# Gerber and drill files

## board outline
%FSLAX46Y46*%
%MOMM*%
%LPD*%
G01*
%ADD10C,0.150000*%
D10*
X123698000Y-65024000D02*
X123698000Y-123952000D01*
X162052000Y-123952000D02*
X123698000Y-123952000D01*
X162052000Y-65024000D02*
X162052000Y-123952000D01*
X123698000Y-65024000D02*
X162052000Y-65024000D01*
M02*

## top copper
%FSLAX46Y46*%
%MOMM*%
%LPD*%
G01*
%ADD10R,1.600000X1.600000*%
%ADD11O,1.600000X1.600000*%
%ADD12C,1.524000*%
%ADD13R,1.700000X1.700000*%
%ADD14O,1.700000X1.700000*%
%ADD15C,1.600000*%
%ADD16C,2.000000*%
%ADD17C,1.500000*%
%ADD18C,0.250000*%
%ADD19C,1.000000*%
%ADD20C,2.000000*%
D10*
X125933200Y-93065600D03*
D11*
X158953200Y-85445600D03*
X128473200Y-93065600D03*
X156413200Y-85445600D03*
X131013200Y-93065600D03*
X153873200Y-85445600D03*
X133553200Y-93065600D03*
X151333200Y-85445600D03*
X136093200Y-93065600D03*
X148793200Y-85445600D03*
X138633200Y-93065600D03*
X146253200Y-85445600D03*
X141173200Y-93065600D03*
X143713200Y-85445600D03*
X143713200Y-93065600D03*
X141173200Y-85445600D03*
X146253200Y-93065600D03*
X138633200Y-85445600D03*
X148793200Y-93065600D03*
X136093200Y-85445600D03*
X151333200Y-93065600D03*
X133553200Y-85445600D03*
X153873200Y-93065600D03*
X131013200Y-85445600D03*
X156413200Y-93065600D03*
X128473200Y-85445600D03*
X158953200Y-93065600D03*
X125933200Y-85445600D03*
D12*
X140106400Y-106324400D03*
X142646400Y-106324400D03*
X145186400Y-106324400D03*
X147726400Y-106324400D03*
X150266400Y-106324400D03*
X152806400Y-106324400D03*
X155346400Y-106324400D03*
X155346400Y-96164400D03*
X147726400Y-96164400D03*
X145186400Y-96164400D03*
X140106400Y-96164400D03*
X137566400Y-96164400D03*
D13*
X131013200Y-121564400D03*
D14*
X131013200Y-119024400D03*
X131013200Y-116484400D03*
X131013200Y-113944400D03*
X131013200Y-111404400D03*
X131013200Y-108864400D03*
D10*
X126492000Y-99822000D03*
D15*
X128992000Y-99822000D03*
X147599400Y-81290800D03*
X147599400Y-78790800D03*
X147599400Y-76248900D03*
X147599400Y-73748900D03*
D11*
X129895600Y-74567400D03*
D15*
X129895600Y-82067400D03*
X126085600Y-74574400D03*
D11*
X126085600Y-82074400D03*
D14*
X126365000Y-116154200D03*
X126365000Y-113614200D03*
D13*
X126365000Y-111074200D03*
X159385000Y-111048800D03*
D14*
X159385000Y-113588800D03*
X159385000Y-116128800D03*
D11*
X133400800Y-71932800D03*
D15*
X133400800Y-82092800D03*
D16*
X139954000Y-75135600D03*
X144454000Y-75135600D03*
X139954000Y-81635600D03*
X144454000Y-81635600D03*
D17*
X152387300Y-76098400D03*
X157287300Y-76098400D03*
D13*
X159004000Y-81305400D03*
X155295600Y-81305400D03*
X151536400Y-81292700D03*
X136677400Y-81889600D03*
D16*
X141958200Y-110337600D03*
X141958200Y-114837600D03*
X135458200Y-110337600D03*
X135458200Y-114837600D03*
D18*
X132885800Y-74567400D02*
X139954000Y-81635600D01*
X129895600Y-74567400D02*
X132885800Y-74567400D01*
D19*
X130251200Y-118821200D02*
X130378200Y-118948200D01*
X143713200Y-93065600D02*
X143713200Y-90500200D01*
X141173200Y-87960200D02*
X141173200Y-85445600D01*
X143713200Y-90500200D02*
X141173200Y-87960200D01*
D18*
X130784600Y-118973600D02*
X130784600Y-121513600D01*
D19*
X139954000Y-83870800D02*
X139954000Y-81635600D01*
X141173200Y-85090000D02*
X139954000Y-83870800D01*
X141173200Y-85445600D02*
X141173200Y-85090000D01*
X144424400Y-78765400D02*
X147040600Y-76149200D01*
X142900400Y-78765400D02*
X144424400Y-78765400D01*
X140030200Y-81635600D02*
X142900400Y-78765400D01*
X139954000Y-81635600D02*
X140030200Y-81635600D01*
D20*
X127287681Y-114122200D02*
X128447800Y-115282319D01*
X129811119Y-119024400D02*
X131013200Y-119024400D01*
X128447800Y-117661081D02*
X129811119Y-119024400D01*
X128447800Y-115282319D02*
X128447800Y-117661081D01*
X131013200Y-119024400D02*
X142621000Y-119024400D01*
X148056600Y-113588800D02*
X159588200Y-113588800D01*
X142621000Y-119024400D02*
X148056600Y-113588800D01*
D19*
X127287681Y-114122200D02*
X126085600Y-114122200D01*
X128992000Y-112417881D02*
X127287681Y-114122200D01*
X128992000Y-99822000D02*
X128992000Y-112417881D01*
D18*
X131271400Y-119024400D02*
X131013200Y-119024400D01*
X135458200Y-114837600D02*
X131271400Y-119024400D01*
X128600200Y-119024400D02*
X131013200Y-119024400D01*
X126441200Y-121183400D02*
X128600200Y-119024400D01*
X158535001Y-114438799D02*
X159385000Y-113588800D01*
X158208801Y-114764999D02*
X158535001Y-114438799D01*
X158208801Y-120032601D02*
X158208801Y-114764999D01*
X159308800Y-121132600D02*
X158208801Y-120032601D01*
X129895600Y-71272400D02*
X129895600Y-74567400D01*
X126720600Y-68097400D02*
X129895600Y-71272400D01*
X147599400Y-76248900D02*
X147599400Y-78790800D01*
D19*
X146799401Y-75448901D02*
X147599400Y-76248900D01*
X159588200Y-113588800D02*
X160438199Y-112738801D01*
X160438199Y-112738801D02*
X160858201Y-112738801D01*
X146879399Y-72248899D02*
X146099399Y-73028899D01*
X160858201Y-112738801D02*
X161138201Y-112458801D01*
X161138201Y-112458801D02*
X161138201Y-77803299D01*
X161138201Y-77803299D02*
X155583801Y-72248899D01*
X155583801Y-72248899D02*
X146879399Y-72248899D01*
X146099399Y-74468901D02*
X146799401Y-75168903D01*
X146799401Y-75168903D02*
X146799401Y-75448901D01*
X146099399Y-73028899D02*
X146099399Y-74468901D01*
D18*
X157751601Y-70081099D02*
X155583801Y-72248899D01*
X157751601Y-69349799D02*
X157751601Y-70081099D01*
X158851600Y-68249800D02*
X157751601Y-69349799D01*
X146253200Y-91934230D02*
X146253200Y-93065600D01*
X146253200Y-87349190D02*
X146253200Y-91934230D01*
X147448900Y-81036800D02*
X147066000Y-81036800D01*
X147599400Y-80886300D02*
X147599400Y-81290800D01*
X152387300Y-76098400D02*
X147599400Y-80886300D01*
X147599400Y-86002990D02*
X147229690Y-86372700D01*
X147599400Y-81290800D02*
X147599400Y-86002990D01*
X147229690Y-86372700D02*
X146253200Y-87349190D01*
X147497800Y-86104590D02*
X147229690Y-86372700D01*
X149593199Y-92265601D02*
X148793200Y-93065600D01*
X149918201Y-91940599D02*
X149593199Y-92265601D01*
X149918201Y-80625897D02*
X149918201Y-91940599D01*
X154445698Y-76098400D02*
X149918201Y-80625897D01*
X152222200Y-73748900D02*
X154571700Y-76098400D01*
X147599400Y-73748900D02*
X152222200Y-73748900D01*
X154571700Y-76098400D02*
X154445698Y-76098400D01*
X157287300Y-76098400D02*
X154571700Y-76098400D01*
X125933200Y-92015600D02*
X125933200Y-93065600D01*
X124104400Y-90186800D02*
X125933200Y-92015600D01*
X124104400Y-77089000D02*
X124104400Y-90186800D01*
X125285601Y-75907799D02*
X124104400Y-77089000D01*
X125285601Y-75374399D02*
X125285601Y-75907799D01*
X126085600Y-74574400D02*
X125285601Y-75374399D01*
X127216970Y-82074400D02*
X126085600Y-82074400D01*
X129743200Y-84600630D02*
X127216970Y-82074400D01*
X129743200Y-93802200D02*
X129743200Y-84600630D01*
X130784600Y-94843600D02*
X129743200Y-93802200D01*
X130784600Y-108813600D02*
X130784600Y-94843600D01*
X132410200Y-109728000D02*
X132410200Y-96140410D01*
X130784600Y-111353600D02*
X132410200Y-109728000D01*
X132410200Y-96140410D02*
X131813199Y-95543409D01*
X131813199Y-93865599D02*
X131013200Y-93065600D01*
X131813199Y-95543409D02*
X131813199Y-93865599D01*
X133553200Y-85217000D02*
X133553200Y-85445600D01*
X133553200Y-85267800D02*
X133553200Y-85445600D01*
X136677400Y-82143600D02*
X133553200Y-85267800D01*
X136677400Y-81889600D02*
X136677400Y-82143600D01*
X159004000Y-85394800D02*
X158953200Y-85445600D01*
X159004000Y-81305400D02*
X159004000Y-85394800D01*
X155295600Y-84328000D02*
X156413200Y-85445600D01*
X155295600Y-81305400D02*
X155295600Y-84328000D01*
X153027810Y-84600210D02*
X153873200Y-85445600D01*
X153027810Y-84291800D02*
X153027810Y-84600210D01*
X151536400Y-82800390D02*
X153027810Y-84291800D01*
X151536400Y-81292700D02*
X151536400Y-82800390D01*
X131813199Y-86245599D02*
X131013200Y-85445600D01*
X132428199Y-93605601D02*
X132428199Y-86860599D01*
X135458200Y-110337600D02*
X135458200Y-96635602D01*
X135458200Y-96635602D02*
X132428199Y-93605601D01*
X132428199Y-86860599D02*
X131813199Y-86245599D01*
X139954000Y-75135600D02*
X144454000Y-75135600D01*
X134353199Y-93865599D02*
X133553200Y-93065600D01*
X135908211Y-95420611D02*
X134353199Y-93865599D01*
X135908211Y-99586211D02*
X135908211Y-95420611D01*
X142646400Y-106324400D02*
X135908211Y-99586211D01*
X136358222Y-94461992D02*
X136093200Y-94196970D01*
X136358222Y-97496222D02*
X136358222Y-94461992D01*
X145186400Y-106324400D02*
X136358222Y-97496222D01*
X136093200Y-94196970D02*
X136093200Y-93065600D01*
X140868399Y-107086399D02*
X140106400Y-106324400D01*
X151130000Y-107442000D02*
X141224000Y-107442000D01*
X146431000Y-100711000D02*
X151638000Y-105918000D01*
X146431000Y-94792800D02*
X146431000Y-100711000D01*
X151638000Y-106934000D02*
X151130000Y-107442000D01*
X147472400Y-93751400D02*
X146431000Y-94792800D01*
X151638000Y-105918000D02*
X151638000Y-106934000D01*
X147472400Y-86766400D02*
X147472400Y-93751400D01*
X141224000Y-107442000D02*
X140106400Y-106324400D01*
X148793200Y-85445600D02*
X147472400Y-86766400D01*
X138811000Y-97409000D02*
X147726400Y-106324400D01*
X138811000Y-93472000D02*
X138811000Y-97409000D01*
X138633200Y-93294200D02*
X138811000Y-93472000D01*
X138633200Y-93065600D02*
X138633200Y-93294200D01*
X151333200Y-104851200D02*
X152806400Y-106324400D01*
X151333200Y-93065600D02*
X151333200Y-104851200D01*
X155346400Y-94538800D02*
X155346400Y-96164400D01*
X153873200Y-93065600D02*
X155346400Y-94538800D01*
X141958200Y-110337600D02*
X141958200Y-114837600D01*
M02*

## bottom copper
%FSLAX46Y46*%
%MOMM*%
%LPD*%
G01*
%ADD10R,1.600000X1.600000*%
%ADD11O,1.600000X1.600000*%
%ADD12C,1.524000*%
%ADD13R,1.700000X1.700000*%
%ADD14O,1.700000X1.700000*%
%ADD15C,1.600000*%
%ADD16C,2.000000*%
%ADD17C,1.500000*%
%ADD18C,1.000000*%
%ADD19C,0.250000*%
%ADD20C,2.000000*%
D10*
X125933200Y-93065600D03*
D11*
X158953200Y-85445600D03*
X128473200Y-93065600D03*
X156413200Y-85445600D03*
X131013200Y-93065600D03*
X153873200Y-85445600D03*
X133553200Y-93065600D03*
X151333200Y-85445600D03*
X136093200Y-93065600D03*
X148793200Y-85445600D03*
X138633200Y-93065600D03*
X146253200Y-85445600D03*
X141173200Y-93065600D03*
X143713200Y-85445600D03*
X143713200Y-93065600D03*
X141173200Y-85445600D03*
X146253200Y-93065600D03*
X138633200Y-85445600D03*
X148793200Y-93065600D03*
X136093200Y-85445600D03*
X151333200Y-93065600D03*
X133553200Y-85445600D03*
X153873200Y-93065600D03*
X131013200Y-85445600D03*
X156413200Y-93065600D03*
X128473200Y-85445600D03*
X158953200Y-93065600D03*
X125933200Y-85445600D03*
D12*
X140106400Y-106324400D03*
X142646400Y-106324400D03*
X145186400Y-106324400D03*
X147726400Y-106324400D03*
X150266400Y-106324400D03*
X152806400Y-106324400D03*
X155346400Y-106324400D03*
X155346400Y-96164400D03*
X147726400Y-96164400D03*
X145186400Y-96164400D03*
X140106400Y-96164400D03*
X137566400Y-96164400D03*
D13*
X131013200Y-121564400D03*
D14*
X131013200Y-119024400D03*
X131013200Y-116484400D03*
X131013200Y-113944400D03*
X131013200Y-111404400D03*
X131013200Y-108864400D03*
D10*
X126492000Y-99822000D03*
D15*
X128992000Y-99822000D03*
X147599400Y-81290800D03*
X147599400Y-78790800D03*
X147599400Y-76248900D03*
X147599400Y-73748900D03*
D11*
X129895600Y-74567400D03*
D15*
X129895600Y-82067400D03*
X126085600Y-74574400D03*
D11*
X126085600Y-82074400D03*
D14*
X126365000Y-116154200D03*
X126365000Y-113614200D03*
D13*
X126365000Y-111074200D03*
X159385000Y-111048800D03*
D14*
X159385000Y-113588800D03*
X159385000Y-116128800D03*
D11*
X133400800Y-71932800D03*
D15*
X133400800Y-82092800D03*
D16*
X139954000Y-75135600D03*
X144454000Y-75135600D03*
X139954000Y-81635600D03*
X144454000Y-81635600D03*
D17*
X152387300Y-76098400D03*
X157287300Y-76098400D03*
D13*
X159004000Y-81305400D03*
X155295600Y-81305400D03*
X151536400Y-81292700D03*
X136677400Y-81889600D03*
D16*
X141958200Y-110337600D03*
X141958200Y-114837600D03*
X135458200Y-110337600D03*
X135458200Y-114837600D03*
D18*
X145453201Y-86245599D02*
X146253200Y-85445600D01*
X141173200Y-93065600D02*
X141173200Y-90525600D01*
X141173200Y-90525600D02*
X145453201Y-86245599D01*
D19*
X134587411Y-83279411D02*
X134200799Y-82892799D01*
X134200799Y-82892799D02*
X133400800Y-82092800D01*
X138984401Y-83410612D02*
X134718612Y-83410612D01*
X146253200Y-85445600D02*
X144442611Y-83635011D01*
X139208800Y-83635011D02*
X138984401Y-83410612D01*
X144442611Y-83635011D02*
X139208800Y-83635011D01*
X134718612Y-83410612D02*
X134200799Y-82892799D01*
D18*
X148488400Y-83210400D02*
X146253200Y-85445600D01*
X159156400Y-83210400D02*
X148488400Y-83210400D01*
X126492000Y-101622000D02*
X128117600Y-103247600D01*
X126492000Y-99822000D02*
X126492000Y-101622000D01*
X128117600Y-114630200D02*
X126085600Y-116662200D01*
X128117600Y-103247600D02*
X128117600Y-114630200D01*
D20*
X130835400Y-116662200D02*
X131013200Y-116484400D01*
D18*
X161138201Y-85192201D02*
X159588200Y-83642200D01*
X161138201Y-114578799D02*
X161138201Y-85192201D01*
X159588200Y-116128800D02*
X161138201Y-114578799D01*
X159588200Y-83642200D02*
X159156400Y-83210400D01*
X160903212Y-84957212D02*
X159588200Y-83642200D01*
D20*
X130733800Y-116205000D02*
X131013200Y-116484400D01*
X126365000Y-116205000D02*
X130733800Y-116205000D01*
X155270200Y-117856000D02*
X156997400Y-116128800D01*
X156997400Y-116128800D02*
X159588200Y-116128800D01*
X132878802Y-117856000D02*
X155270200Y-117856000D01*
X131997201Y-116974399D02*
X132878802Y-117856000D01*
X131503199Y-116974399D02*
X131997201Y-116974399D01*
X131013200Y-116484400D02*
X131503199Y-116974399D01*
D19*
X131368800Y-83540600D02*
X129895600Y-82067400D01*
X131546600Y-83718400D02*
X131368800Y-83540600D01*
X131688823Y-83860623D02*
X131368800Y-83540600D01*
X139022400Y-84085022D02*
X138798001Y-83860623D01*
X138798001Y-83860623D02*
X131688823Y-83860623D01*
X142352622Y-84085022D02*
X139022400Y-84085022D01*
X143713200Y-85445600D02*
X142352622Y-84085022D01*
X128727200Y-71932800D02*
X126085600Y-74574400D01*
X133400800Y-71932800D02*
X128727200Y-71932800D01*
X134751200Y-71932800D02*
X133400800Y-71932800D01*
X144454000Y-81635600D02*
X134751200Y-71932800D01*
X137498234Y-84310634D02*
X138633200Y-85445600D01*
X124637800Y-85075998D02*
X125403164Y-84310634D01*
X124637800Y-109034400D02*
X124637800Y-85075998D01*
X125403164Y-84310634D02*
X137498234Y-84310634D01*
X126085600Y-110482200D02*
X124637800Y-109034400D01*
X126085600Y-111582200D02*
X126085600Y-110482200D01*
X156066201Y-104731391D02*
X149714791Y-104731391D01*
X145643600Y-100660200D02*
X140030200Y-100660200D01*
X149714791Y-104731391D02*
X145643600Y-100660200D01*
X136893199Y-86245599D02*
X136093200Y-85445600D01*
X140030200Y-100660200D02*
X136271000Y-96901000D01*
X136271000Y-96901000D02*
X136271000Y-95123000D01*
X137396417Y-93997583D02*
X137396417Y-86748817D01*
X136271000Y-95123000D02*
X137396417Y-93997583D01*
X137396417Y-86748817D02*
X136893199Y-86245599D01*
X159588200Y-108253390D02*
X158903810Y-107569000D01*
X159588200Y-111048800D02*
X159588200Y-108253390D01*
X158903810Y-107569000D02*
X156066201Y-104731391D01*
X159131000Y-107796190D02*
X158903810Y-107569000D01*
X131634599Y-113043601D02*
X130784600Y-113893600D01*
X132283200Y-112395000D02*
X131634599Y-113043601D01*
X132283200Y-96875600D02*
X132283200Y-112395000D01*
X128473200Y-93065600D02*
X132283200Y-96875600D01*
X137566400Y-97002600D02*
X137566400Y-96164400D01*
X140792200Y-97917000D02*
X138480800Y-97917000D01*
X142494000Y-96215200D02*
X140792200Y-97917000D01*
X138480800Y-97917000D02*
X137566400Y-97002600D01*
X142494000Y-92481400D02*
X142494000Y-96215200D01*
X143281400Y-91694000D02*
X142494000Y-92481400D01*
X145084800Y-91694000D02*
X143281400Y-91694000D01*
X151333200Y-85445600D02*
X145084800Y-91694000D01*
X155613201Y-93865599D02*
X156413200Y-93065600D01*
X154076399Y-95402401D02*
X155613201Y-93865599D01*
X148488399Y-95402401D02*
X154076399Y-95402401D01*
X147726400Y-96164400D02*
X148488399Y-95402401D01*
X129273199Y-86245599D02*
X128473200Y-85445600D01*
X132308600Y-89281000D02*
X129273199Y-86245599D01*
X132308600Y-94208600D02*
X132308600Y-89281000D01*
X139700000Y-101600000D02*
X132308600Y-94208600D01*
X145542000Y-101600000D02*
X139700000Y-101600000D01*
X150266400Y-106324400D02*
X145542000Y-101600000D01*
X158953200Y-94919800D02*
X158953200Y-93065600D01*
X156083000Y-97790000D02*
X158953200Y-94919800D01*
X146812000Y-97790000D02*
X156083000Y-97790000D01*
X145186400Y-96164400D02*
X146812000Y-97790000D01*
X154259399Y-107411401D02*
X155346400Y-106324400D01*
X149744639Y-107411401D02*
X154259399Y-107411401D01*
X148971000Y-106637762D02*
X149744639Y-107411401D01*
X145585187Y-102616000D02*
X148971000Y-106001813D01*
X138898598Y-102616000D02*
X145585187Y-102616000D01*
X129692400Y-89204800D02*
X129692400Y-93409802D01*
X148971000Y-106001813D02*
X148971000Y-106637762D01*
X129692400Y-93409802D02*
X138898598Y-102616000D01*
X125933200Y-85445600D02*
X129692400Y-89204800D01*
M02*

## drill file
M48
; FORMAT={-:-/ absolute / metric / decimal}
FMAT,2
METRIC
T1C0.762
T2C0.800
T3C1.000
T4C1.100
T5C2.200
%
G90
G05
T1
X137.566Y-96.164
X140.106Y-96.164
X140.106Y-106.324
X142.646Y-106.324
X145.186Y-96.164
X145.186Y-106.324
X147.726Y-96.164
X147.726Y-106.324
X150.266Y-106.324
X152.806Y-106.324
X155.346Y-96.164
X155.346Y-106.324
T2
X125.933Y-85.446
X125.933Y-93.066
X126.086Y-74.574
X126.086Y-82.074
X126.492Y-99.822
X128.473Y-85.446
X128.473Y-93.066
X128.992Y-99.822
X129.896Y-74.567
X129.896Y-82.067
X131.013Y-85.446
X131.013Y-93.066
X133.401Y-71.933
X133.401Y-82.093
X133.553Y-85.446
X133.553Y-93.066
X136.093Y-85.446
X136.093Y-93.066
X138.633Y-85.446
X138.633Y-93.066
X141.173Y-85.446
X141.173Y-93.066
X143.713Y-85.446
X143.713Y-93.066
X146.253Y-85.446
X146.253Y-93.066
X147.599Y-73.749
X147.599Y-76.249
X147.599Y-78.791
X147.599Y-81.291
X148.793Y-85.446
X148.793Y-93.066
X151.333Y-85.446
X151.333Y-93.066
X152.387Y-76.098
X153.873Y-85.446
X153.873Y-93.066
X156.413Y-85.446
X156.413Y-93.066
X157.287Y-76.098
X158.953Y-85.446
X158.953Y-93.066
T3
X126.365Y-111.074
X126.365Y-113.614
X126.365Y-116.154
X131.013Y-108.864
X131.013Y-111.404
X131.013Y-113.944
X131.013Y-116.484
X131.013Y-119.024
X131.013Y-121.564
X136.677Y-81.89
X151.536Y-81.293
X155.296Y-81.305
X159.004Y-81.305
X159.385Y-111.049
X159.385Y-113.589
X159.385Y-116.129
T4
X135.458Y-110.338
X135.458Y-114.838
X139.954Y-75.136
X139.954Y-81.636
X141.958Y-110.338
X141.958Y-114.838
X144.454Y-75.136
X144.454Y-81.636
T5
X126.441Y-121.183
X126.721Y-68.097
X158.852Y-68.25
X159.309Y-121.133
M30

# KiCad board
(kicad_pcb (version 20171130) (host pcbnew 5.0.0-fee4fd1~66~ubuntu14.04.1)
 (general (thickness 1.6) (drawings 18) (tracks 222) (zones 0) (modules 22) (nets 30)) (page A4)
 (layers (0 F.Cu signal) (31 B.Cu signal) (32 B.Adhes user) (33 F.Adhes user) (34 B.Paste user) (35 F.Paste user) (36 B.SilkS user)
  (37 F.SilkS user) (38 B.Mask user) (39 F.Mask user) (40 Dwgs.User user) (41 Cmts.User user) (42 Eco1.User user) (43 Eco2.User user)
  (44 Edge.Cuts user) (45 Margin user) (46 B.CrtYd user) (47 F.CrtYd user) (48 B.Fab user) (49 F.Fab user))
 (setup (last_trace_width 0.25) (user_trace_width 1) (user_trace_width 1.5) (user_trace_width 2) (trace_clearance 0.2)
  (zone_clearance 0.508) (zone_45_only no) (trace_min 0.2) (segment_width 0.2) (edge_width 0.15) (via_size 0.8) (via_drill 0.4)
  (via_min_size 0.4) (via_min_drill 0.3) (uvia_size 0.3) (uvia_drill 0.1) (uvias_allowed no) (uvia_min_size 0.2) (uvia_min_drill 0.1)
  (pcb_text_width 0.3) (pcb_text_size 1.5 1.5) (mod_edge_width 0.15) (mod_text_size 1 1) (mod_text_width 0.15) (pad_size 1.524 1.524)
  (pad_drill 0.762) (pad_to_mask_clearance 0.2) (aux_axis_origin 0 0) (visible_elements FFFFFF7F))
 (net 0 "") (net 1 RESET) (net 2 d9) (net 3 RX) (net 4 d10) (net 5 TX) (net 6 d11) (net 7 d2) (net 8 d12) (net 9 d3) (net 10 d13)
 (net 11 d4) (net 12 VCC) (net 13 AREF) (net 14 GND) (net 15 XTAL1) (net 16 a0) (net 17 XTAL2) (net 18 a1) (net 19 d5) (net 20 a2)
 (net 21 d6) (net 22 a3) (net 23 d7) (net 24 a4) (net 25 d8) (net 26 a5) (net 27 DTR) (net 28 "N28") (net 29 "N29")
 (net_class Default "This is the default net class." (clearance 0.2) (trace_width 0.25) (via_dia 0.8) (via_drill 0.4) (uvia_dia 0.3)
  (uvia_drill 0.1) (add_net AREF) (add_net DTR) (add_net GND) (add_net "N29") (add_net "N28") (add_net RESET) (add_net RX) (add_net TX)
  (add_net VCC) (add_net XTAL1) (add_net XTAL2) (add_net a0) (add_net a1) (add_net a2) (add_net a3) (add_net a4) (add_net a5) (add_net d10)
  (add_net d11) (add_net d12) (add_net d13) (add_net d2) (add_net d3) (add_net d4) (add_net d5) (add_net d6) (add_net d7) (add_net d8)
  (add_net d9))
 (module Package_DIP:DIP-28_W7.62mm (layer F.Cu) (at 125.9332 93.0656 90)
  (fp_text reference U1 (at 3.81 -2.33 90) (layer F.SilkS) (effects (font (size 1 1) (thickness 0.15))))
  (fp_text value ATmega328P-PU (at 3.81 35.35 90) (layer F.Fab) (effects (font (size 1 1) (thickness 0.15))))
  (pad 1 thru_hole rect (at 0 0 90) (size 1.6 1.6) (drill 0.8) (layers *.Cu *.Mask) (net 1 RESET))
  (pad 15 thru_hole oval (at 7.62 33.02 90) (size 1.6 1.6) (drill 0.8) (layers *.Cu *.Mask) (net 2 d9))
  (pad 2 thru_hole oval (at 0 2.54 90) (size 1.6 1.6) (drill 0.8) (layers *.Cu *.Mask) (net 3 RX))
  (pad 16 thru_hole oval (at 7.62 30.48 90) (size 1.6 1.6) (drill 0.8) (layers *.Cu *.Mask) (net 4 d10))
  (pad 3 thru_hole oval (at 0 5.08 90) (size 1.6 1.6) (drill 0.8) (layers *.Cu *.Mask) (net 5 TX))
  (pad 17 thru_hole oval (at 7.62 27.94 90) (size 1.6 1.6) (drill 0.8) (layers *.Cu *.Mask) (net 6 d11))
  (pad 4 thru_hole oval (at 0 7.62 90) (size 1.6 1.6) (drill 0.8) (layers *.Cu *.Mask) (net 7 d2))
  (pad 18 thru_hole oval (at 7.62 25.4 90) (size 1.6 1.6) (drill 0.8) (layers *.Cu *.Mask) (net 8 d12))
  (pad 5 thru_hole oval (at 0 10.16 90) (size 1.6 1.6) (drill 0.8) (layers *.Cu *.Mask) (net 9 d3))
  (pad 19 thru_hole oval (at 7.62 22.86 90) (size 1.6 1.6) (drill 0.8) (layers *.Cu *.Mask) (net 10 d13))
  (pad 6 thru_hole oval (at 0 12.7 90) (size 1.6 1.6) (drill 0.8) (layers *.Cu *.Mask) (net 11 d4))
  (pad 20 thru_hole oval (at 7.62 20.32 90) (size 1.6 1.6) (drill 0.8) (layers *.Cu *.Mask) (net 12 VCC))
  (pad 7 thru_hole oval (at 0 15.24 90) (size 1.6 1.6) (drill 0.8) (layers *.Cu *.Mask) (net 12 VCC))
  (pad 21 thru_hole oval (at 7.62 17.78 90) (size 1.6 1.6) (drill 0.8) (layers *.Cu *.Mask) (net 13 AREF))
  (pad 8 thru_hole oval (at 0 17.78 90) (size 1.6 1.6) (drill 0.8) (layers *.Cu *.Mask) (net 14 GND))
  (pad 22 thru_hole oval (at 7.62 15.24 90) (size 1.6 1.6) (drill 0.8) (layers *.Cu *.Mask) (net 14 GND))
  (pad 9 thru_hole oval (at 0 20.32 90) (size 1.6 1.6) (drill 0.8) (layers *.Cu *.Mask) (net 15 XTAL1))
  (pad 23 thru_hole oval (at 7.62 12.7 90) (size 1.6 1.6) (drill 0.8) (layers *.Cu *.Mask) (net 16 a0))
  (pad 10 thru_hole oval (at 0 22.86 90) (size 1.6 1.6) (drill 0.8) (layers *.Cu *.Mask) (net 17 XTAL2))
  (pad 24 thru_hole oval (at 7.62 10.16 90) (size 1.6 1.6) (drill 0.8) (layers *.Cu *.Mask) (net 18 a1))
  (pad 11 thru_hole oval (at 0 25.4 90) (size 1.6 1.6) (drill 0.8) (layers *.Cu *.Mask) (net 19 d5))
  (pad 25 thru_hole oval (at 7.62 7.62 90) (size 1.6 1.6) (drill 0.8) (layers *.Cu *.Mask) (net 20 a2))
  (pad 12 thru_hole oval (at 0 27.94 90) (size 1.6 1.6) (drill 0.8) (layers *.Cu *.Mask) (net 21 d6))
  (pad 26 thru_hole oval (at 7.62 5.08 90) (size 1.6 1.6) (drill 0.8) (layers *.Cu *.Mask) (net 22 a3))
  (pad 13 thru_hole oval (at 0 30.48 90) (size 1.6 1.6) (drill 0.8) (layers *.Cu *.Mask) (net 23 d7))
  (pad 27 thru_hole oval (at 7.62 2.54 90) (size 1.6 1.6) (drill 0.8) (layers *.Cu *.Mask) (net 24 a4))
  (pad 14 thru_hole oval (at 0 33.02 90) (size 1.6 1.6) (drill 0.8) (layers *.Cu *.Mask) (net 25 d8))
  (pad 28 thru_hole oval (at 7.62 0 90) (size 1.6 1.6) (drill 0.8) (layers *.Cu *.Mask) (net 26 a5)))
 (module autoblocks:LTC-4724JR (layer F.Cu) (at 147.7264 102.5144)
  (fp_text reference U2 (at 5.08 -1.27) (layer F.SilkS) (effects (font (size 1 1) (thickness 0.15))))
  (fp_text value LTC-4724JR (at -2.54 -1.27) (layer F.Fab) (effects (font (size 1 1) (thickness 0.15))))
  (pad 1 thru_hole circle (at -7.62 3.81) (size 1.524 1.524) (drill 0.762) (layers *.Cu *.Mask) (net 10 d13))
  (pad 2 thru_hole circle (at -5.08 3.81) (size 1.524 1.524) (drill 0.762) (layers *.Cu *.Mask) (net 7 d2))
  (pad 3 thru_hole circle (at -2.54 3.81) (size 1.524 1.524) (drill 0.762) (layers *.Cu *.Mask) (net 9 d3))
  (pad 4 thru_hole circle (at 0 3.81) (size 1.524 1.524) (drill 0.762) (layers *.Cu *.Mask) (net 11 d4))
  (pad 5 thru_hole circle (at 2.54 3.81) (size 1.524 1.524) (drill 0.762) (layers *.Cu *.Mask) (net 24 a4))
  (pad 6 thru_hole circle (at 5.08 3.81) (size 1.524 1.524) (drill 0.762) (layers *.Cu *.Mask) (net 19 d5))
  (pad 7 thru_hole circle (at 7.62 3.81) (size 1.524 1.524) (drill 0.762) (layers *.Cu *.Mask) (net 26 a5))
  (pad 8 thru_hole circle (at 7.62 -6.35) (size 1.524 1.524) (drill 0.762) (layers *.Cu *.Mask) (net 21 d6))
  (pad 11 thru_hole circle (at 0 -6.35) (size 1.524 1.524) (drill 0.762) (layers *.Cu *.Mask) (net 23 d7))
  (pad 12 thru_hole circle (at -2.54 -6.35) (size 1.524 1.524) (drill 0.762) (layers *.Cu *.Mask) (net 25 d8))
  (pad 14 thru_hole circle (at -7.62 -6.35) (size 1.524 1.524) (drill 0.762) (layers *.Cu *.Mask))
  (pad 15 thru_hole circle (at -10.16 -6.35) (size 1.524 1.524) (drill 0.762) (layers *.Cu *.Mask) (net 8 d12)))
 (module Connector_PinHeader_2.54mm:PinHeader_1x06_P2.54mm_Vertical (layer F.Cu) (at 131.0132 121.5644 180)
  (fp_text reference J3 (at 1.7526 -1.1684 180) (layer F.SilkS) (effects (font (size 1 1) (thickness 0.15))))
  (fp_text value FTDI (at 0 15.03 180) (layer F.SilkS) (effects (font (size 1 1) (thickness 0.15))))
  (pad 1 thru_hole rect (at 0 0 180) (size 1.7 1.7) (drill 1) (layers *.Cu *.Mask) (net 14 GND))
  (pad 2 thru_hole oval (at 0 2.54 180) (size 1.7 1.7) (drill 1) (layers *.Cu *.Mask) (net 14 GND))
  (pad 3 thru_hole oval (at 0 5.08 180) (size 1.7 1.7) (drill 1) (layers *.Cu *.Mask) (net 12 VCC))
  (pad 4 thru_hole oval (at 0 7.62 180) (size 1.7 1.7) (drill 1) (layers *.Cu *.Mask) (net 3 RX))
  (pad 5 thru_hole oval (at 0 10.16 180) (size 1.7 1.7) (drill 1) (layers *.Cu *.Mask) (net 5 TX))
  (pad 6 thru_hole oval (at 0 12.7 180) (size 1.7 1.7) (drill 1) (layers *.Cu *.Mask) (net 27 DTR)))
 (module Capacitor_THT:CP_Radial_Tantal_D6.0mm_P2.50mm (layer F.Cu) (at 126.492 99.822)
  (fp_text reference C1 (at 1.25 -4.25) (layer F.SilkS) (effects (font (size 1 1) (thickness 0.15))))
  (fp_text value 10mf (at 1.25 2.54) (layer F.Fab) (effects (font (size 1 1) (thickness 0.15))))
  (pad 1 thru_hole rect (at 0 0) (size 1.6 1.6) (drill 0.8) (layers *.Cu *.Mask) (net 12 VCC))
  (pad 2 thru_hole circle (at 2.5 0) (size 1.6 1.6) (drill 0.8) (layers *.Cu *.Mask) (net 14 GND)))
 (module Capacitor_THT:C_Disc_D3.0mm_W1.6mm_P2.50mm (layer F.Cu) (at 147.5994 78.7908 270)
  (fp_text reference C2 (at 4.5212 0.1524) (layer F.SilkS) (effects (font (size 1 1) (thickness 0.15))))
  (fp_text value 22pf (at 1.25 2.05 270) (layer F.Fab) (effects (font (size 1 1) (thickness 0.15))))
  (pad 2 thru_hole circle (at 2.5 0 270) (size 1.6 1.6) (drill 0.8) (layers *.Cu *.Mask) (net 15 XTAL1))
  (pad 1 thru_hole circle (at 0 0 270) (size 1.6 1.6) (drill 0.8) (layers *.Cu *.Mask) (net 14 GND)))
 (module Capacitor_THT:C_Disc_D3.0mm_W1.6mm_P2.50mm (layer F.Cu) (at 147.5994 76.2489 90)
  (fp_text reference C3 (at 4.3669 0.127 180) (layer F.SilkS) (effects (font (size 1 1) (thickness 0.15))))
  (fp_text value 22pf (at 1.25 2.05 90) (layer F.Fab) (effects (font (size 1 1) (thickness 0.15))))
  (pad 1 thru_hole circle (at 0 0 90) (size 1.6 1.6) (drill 0.8) (layers *.Cu *.Mask) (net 14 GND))
  (pad 2 thru_hole circle (at 2.5 0 90) (size 1.6 1.6) (drill 0.8) (layers *.Cu *.Mask) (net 17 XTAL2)))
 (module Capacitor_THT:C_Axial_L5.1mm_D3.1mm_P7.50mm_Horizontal (layer F.Cu) (at 129.8956 82.0674 90)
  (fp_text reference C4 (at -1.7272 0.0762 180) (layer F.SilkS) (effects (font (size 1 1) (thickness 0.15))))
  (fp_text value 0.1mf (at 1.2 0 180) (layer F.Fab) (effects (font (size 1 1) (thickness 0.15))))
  (pad 2 thru_hole oval (at 7.5 0 90) (size 1.6 1.6) (drill 0.8) (layers *.Cu *.Mask) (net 14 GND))
  (pad 1 thru_hole circle (at 0 0 90) (size 1.6 1.6) (drill 0.8) (layers *.Cu *.Mask) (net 13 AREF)))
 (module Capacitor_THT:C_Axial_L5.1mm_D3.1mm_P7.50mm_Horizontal (layer F.Cu) (at 126.0856 74.5744 270)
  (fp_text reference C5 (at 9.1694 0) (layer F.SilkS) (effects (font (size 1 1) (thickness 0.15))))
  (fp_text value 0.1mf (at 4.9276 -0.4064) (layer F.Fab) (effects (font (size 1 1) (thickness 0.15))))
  (pad 1 thru_hole circle (at 0 0 270) (size 1.6 1.6) (drill 0.8) (layers *.Cu *.Mask) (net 1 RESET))
  (pad 2 thru_hole oval (at 7.5 0 270) (size 1.6 1.6) (drill 0.8) (layers *.Cu *.Mask) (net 27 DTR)))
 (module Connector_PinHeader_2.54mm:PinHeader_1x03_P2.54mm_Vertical (layer F.Cu) (at 126.365 111.0742)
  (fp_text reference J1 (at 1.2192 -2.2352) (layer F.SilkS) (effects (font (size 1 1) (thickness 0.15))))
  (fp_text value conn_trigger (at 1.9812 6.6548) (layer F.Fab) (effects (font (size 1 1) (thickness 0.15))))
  (pad 3 thru_hole oval (at 0 5.08) (size 1.7 1.7) (drill 1) (layers *.Cu *.Mask) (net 12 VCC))
  (pad 2 thru_hole oval (at 0 2.54) (size 1.7 1.7) (drill 1) (layers *.Cu *.Mask) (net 14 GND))
  (pad 1 thru_hole rect (at 0 0) (size 1.7 1.7) (drill 1) (layers *.Cu *.Mask) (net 16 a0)))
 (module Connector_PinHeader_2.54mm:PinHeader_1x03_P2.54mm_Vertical (layer F.Cu) (at 159.385 111.0488)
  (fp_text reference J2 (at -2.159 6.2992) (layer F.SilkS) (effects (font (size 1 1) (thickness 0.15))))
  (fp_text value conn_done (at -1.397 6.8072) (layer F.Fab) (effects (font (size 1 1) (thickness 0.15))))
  (pad 1 thru_hole rect (at 0 0) (size 1.7 1.7) (drill 1) (layers *.Cu *.Mask) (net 18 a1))
  (pad 2 thru_hole oval (at 0 2.54) (size 1.7 1.7) (drill 1) (layers *.Cu *.Mask) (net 14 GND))
  (pad 3 thru_hole oval (at 0 5.08) (size 1.7 1.7) (drill 1) (layers *.Cu *.Mask) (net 12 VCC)))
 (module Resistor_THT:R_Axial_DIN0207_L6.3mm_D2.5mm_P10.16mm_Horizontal (layer F.Cu) (at 133.4008 82.0928 90)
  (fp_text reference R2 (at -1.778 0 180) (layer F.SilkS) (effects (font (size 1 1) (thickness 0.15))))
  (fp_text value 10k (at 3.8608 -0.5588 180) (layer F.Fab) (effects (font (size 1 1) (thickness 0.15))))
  (pad 2 thru_hole oval (at 10.16 0 90) (size 1.6 1.6) (drill 0.8) (layers *.Cu *.Mask) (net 1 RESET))
  (pad 1 thru_hole circle (at 0 0 90) (size 1.6 1.6) (drill 0.8) (layers *.Cu *.Mask) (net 12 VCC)))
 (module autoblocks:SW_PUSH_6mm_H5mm (layer F.Cu) (at 139.954 81.6356 90)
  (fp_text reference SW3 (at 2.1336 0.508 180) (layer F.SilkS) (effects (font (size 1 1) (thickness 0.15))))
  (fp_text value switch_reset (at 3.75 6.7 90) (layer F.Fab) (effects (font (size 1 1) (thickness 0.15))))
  (pad 3 thru_hole circle (at 6.5 0 180) (size 2 2) (drill 1.1) (layers *.Cu *.Mask) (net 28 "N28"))
  (pad 4 thru_hole circle (at 6.5 4.5 180) (size 2 2) (drill 1.1) (layers *.Cu *.Mask) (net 28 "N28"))
  (pad 1 thru_hole circle (at 0 0 180) (size 2 2) (drill 1.1) (layers *.Cu *.Mask) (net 14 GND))
  (pad 2 thru_hole circle (at 0 4.5 180) (size 2 2) (drill 1.1) (layers *.Cu *.Mask) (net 1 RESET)))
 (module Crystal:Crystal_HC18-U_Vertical (layer F.Cu) (at 152.3873 76.0984)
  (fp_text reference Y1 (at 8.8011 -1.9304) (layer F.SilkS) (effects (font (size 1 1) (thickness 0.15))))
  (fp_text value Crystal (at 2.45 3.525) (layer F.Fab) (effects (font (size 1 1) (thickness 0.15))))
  (pad 1 thru_hole circle (at 0 0) (size 1.5 1.5) (drill 0.8) (layers *.Cu *.Mask) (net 15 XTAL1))
  (pad 2 thru_hole circle (at 4.9 0) (size 1.5 1.5) (drill 0.8) (layers *.Cu *.Mask) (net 17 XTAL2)))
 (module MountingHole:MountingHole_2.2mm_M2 (layer F.Cu) (at 126.7206 68.0974)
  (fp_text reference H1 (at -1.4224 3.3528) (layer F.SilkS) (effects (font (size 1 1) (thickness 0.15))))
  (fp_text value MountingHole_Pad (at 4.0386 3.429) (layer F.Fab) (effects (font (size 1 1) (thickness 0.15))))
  (pad 1 np_thru_hole circle (at 0 0) (size 2.2 2.2) (drill 2.2) (layers *.Cu *.Mask) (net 14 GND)))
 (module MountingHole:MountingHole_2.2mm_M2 (layer F.Cu) (at 158.8516 68.2498)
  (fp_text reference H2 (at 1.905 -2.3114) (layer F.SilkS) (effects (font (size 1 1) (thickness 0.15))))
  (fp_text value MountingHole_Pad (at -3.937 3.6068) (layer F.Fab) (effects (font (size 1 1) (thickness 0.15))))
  (pad 1 np_thru_hole circle (at 0 0) (size 2.2 2.2) (drill 2.2) (layers *.Cu *.Mask) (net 14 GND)))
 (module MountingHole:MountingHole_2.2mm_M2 (layer F.Cu) (at 126.4412 121.1834)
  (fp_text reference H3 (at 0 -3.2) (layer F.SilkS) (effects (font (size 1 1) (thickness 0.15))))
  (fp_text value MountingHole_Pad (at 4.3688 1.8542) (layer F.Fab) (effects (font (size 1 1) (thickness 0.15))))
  (pad 1 np_thru_hole circle (at 0 0) (size 2.2 2.2) (drill 2.2) (layers *.Cu *.Mask) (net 14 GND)))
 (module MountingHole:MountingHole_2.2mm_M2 (layer F.Cu) (at 159.3088 121.1326)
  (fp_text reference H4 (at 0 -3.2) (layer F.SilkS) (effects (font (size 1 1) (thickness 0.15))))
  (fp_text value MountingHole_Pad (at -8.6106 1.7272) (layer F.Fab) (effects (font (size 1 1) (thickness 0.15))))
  (pad 1 np_thru_hole circle (at 0 0) (size 2.2 2.2) (drill 2.2) (layers *.Cu *.Mask) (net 14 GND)))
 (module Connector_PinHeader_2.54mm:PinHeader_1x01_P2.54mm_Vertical (layer F.Cu) (at 159.004 81.3054)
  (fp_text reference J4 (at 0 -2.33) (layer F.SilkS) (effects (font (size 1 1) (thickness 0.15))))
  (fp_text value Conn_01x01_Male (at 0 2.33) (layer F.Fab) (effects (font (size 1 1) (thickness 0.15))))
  (pad 1 thru_hole rect (at 0 0) (size 1.7 1.7) (drill 1) (layers *.Cu *.Mask) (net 2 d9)))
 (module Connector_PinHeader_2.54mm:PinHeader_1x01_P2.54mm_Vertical (layer F.Cu) (at 155.2956 81.3054)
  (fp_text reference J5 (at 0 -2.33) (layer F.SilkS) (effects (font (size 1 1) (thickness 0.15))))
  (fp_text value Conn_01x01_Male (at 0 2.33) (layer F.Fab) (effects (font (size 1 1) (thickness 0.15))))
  (pad 1 thru_hole rect (at 0 0) (size 1.7 1.7) (drill 1) (layers *.Cu *.Mask) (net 4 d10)))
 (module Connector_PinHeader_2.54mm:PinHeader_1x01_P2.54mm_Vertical (layer F.Cu) (at 151.5364 81.2927)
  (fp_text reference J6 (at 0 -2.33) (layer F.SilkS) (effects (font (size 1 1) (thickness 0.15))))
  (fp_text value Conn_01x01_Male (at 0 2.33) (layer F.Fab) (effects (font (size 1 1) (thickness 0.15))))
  (pad 1 thru_hole rect (at 0 0) (size 1.7 1.7) (drill 1) (layers *.Cu *.Mask) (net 6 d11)))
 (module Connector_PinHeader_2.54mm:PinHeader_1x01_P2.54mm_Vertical (layer F.Cu) (at 136.6774 81.8896)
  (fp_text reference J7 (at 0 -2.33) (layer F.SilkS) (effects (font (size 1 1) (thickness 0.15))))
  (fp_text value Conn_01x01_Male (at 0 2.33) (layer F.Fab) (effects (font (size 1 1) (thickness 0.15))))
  (pad 1 thru_hole rect (at 0 0) (size 1.7 1.7) (drill 1) (layers *.Cu *.Mask) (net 20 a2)))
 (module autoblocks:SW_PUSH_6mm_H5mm (layer F.Cu) (at 135.4582 110.3376)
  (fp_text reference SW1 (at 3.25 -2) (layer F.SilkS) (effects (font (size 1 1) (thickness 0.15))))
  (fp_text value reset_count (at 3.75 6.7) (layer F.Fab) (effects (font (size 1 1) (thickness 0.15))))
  (pad 3 thru_hole circle (at 6.5 0 90) (size 2 2) (drill 1.1) (layers *.Cu *.Mask) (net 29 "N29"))
  (pad 4 thru_hole circle (at 6.5 4.5 90) (size 2 2) (drill 1.1) (layers *.Cu *.Mask) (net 29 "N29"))
  (pad 1 thru_hole circle (at 0 0 90) (size 2 2) (drill 1.1) (layers *.Cu *.Mask) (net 22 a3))
  (pad 2 thru_hole circle (at 0 4.5 90) (size 2 2) (drill 1.1) (layers *.Cu *.Mask) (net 14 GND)))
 (gr_line (start 123.698 65.024) (end 123.698 123.952) (layer Edge.Cuts) (width 0.15))
 (gr_line (start 162.052 123.952) (end 123.698 123.952) (layer Edge.Cuts) (width 0.15))
 (gr_line (start 162.052 65.024) (end 162.052 123.952) (layer Edge.Cuts) (width 0.15))
 (gr_line (start 123.698 65.024) (end 162.052 65.024) (layer Edge.Cuts) (width 0.15))
 (segment (start 132.8858 74.5674) (end 139.954 81.6356) (width 0.25) (layer F.Cu) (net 14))
 (segment (start 129.8956 74.5674) (end 132.8858 74.5674) (width 0.25) (layer F.Cu) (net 14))
 (segment (start 130.2512 118.8212) (end 130.3782 118.9482) (width 1) (layer F.Cu) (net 14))
 (segment (start 143.7132 93.0656) (end 143.7132 90.5002) (width 1) (layer F.Cu) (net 14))
 (segment (start 141.1732 87.9602) (end 141.1732 85.4456) (width 1) (layer F.Cu) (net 14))
 (segment (start 143.7132 90.5002) (end 141.1732 87.9602) (width 1) (layer F.Cu) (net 14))
 (segment (start 130.7846 118.9736) (end 130.7846 121.5136) (width 0.25) (layer F.Cu) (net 14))
 (segment (start 139.954 83.8708) (end 139.954 81.6356) (width 1) (layer F.Cu) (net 14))
 (segment (start 141.1732 85.09) (end 139.954 83.8708) (width 1) (layer F.Cu) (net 14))
 (segment (start 141.1732 85.4456) (end 141.1732 85.09) (width 1) (layer F.Cu) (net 14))
 (segment (start 144.4244 78.7654) (end 147.0406 76.1492) (width 1) (layer F.Cu) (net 14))
 (segment (start 142.9004 78.7654) (end 144.4244 78.7654) (width 1) (layer F.Cu) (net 14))
 (segment (start 140.0302 81.6356) (end 142.9004 78.7654) (width 1) (layer F.Cu) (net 14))
 (segment (start 139.954 81.6356) (end 140.0302 81.6356) (width 1) (layer F.Cu) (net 14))
 (segment (start 127.287681 114.1222) (end 128.4478 115.282319) (width 2) (layer F.Cu) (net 14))
 (segment (start 129.811119 119.0244) (end 131.0132 119.0244) (width 2) (layer F.Cu) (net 14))
 (segment (start 128.4478 117.661081) (end 129.811119 119.0244) (width 2) (layer F.Cu) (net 14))
 (segment (start 128.4478 115.282319) (end 128.4478 117.661081) (width 2) (layer F.Cu) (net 14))
 (segment (start 131.0132 119.0244) (end 142.621 119.0244) (width 2) (layer F.Cu) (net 14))
 (segment (start 148.0566 113.5888) (end 159.5882 113.5888) (width 2) (layer F.Cu) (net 14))
 (segment (start 142.621 119.0244) (end 148.0566 113.5888) (width 2) (layer F.Cu) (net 14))
 (segment (start 127.287681 114.1222) (end 126.0856 114.1222) (width 1) (layer F.Cu) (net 14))
 (segment (start 128.992 112.417881) (end 127.287681 114.1222) (width 1) (layer F.Cu) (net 14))
 (segment (start 128.992 99.822) (end 128.992 112.417881) (width 1) (layer F.Cu) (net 14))
 (segment (start 131.2714 119.0244) (end 131.0132 119.0244) (width 0.25) (layer F.Cu) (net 14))
 (segment (start 135.4582 114.8376) (end 131.2714 119.0244) (width 0.25) (layer F.Cu) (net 14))
 (segment (start 128.6002 119.0244) (end 131.0132 119.0244) (width 0.25) (layer F.Cu) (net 14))
 (segment (start 126.4412 121.1834) (end 128.6002 119.0244) (width 0.25) (layer F.Cu) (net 14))
 (segment (start 158.535001 114.438799) (end 159.385 113.5888) (width 0.25) (layer F.Cu) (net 14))
 (segment (start 158.208801 114.764999) (end 158.535001 114.438799) (width 0.25) (layer F.Cu) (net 14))
 (segment (start 158.208801 120.032601) (end 158.208801 114.764999) (width 0.25) (layer F.Cu) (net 14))
 (segment (start 159.3088 121.1326) (end 158.208801 120.032601) (width 0.25) (layer F.Cu) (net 14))
 (segment (start 129.8956 71.2724) (end 129.8956 74.5674) (width 0.25) (layer F.Cu) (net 14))
 (segment (start 126.7206 68.0974) (end 129.8956 71.2724) (width 0.25) (layer F.Cu) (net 14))
 (segment (start 147.5994 76.2489) (end 147.5994 78.7908) (width 0.25) (layer F.Cu) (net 14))
 (segment (start 146.799401 75.448901) (end 147.5994 76.2489) (width 1) (layer F.Cu) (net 14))
 (segment (start 159.5882 113.5888) (end 160.438199 112.738801) (width 1) (layer F.Cu) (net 14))
 (segment (start 160.438199 112.738801) (end 160.858201 112.738801) (width 1) (layer F.Cu) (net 14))
 (segment (start 146.879399 72.248899) (end 146.099399 73.028899) (width 1) (layer F.Cu) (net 14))
 (segment (start 160.858201 112.738801) (end 161.138201 112.458801) (width 1) (layer F.Cu) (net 14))
 (segment (start 161.138201 112.458801) (end 161.138201 77.803299) (width 1) (layer F.Cu) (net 14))
 (segment (start 161.138201 77.803299) (end 155.583801 72.248899) (width 1) (layer F.Cu) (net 14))
 (segment (start 155.583801 72.248899) (end 146.879399 72.248899) (width 1) (layer F.Cu) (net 14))
 (segment (start 146.099399 74.468901) (end 146.799401 75.168903) (width 1) (layer F.Cu) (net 14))
 (segment (start 146.799401 75.168903) (end 146.799401 75.448901) (width 1) (layer F.Cu) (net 14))
 (segment (start 146.099399 73.028899) (end 146.099399 74.468901) (width 1) (layer F.Cu) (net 14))
 (segment (start 157.751601 70.081099) (end 155.583801 72.248899) (width 0.25) (layer F.Cu) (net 14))
 (segment (start 157.751601 69.349799) (end 157.751601 70.081099) (width 0.25) (layer F.Cu) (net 14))
 (segment (start 158.8516 68.2498) (end 157.751601 69.349799) (width 0.25) (layer F.Cu) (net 14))
 (segment (start 145.453201 86.245599) (end 146.2532 85.4456) (width 1) (layer B.Cu) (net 12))
 (segment (start 141.1732 93.0656) (end 141.1732 90.5256) (width 1) (layer B.Cu) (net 12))
 (segment (start 141.1732 90.5256) (end 145.453201 86.245599) (width 1) (layer B.Cu) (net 12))
 (segment (start 134.587411 83.279411) (end 134.200799 82.892799) (width 0.25) (layer B.Cu) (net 12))
 (segment (start 134.200799 82.892799) (end 133.4008 82.0928) (width 0.25) (layer B.Cu) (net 12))
 (segment (start 138.984401 83.410612) (end 134.718612 83.410612) (width 0.25) (layer B.Cu) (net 12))
 (segment (start 146.2532 85.4456) (end 144.442611 83.635011) (width 0.25) (layer B.Cu) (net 12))
 (segment (start 139.2088 83.635011) (end 138.984401 83.410612) (width 0.25) (layer B.Cu) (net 12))
 (segment (start 144.442611 83.635011) (end 139.2088 83.635011) (width 0.25) (layer B.Cu) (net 12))
 (segment (start 134.718612 83.410612) (end 134.200799 82.892799) (width 0.25) (layer B.Cu) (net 12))
 (segment (start 148.4884 83.2104) (end 146.2532 85.4456) (width 1) (layer B.Cu) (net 12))
 (segment (start 159.1564 83.2104) (end 148.4884 83.2104) (width 1) (layer B.Cu) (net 12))
 (segment (start 126.492 101.622) (end 128.1176 103.2476) (width 1) (layer B.Cu) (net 12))
 (segment (start 126.492 99.822) (end 126.492 101.622) (width 1) (layer B.Cu) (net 12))
 (segment (start 128.1176 114.6302) (end 126.0856 116.6622) (width 1) (layer B.Cu) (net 12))
 (segment (start 128.1176 103.2476) (end 128.1176 114.6302) (width 1) (layer B.Cu) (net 12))
 (segment (start 130.8354 116.6622) (end 131.0132 116.4844) (width 2) (layer B.Cu) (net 12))
 (segment (start 161.138201 85.192201) (end 159.5882 83.6422) (width 1) (layer B.Cu) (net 12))
 (segment (start 161.138201 114.578799) (end 161.138201 85.192201) (width 1) (layer B.Cu) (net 12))
 (segment (start 159.5882 116.1288) (end 161.138201 114.578799) (width 1) (layer B.Cu) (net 12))
 (segment (start 159.5882 83.6422) (end 159.1564 83.2104) (width 1) (layer B.Cu) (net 12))
 (segment (start 160.903212 84.957212) (end 159.5882 83.6422) (width 1) (layer B.Cu) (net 12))
 (segment (start 130.7338 116.205) (end 131.0132 116.4844) (width 2) (layer B.Cu) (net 12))
 (segment (start 126.365 116.205) (end 130.7338 116.205) (width 2) (layer B.Cu) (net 12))
 (segment (start 155.2702 117.856) (end 156.9974 116.1288) (width 2) (layer B.Cu) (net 12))
 (segment (start 156.9974 116.1288) (end 159.5882 116.1288) (width 2) (layer B.Cu) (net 12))
 (segment (start 132.878802 117.856) (end 155.2702 117.856) (width 2) (layer B.Cu) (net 12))
 (segment (start 131.997201 116.974399) (end 132.878802 117.856) (width 2) (layer B.Cu) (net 12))
 (segment (start 131.503199 116.974399) (end 131.997201 116.974399) (width 2) (layer B.Cu) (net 12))
 (segment (start 131.0132 116.4844) (end 131.503199 116.974399) (width 2) (layer B.Cu) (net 12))
 (segment (start 146.2532 91.93423) (end 146.2532 93.0656) (width 0.25) (layer F.Cu) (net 15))
 (segment (start 146.2532 87.34919) (end 146.2532 91.93423) (width 0.25) (layer F.Cu) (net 15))
 (segment (start 147.4489 81.0368) (end 147.066 81.0368) (width 0.25) (layer F.Cu) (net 15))
 (segment (start 147.5994 80.8863) (end 147.5994 81.2908) (width 0.25) (layer F.Cu) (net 15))
 (segment (start 152.3873 76.0984) (end 147.5994 80.8863) (width 0.25) (layer F.Cu) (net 15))
 (segment (start 147.5994 86.00299) (end 147.22969 86.3727) (width 0.25) (layer F.Cu) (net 15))
 (segment (start 147.5994 81.2908) (end 147.5994 86.00299) (width 0.25) (layer F.Cu) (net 15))
 (segment (start 147.22969 86.3727) (end 146.2532 87.34919) (width 0.25) (layer F.Cu) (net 15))
 (segment (start 147.4978 86.10459) (end 147.22969 86.3727) (width 0.25) (layer F.Cu) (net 15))
 (segment (start 149.593199 92.265601) (end 148.7932 93.0656) (width 0.25) (layer F.Cu) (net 17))
 (segment (start 149.918201 91.940599) (end 149.593199 92.265601) (width 0.25) (layer F.Cu) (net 17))
 (segment (start 149.918201 80.625897) (end 149.918201 91.940599) (width 0.25) (layer F.Cu) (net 17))
 (segment (start 154.445698 76.0984) (end 149.918201 80.625897) (width 0.25) (layer F.Cu) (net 17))
 (segment (start 152.2222 73.7489) (end 154.5717 76.0984) (width 0.25) (layer F.Cu) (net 17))
 (segment (start 147.5994 73.7489) (end 152.2222 73.7489) (width 0.25) (layer F.Cu) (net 17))
 (segment (start 154.5717 76.0984) (end 154.445698 76.0984) (width 0.25) (layer F.Cu) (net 17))
 (segment (start 157.2873 76.0984) (end 154.5717 76.0984) (width 0.25) (layer F.Cu) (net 17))
 (segment (start 131.3688 83.5406) (end 129.8956 82.0674) (width 0.25) (layer B.Cu) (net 13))
 (segment (start 131.5466 83.7184) (end 131.3688 83.5406) (width 0.25) (layer B.Cu) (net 13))
 (segment (start 131.688823 83.860623) (end 131.3688 83.5406) (width 0.25) (layer B.Cu) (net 13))
 (segment (start 139.0224 84.085022) (end 138.798001 83.860623) (width 0.25) (layer B.Cu) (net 13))
 (segment (start 138.798001 83.860623) (end 131.688823 83.860623) (width 0.25) (layer B.Cu) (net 13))
 (segment (start 142.352622 84.085022) (end 139.0224 84.085022) (width 0.25) (layer B.Cu) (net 13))
 (segment (start 143.7132 85.4456) (end 142.352622 84.085022) (width 0.25) (layer B.Cu) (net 13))
 (segment (start 128.7272 71.9328) (end 126.0856 74.5744) (width 0.25) (layer B.Cu) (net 1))
 (segment (start 133.4008 71.9328) (end 128.7272 71.9328) (width 0.25) (layer B.Cu) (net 1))
 (segment (start 134.7512 71.9328) (end 133.4008 71.9328) (width 0.25) (layer B.Cu) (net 1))
 (segment (start 144.454 81.6356) (end 134.7512 71.9328) (width 0.25) (layer B.Cu) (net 1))
 (segment (start 125.9332 92.0156) (end 125.9332 93.0656) (width 0.25) (layer F.Cu) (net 1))
 (segment (start 124.1044 90.1868) (end 125.9332 92.0156) (width 0.25) (layer F.Cu) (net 1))
 (segment (start 124.1044 77.089) (end 124.1044 90.1868) (width 0.25) (layer F.Cu) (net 1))
 (segment (start 125.285601 75.907799) (end 124.1044 77.089) (width 0.25) (layer F.Cu) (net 1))
 (segment (start 125.285601 75.374399) (end 125.285601 75.907799) (width 0.25) (layer F.Cu) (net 1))
 (segment (start 126.0856 74.5744) (end 125.285601 75.374399) (width 0.25) (layer F.Cu) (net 1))
 (segment (start 127.21697 82.0744) (end 126.0856 82.0744) (width 0.25) (layer F.Cu) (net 27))
 (segment (start 129.7432 84.60063) (end 127.21697 82.0744) (width 0.25) (layer F.Cu) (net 27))
 (segment (start 129.7432 93.8022) (end 129.7432 84.60063) (width 0.25) (layer F.Cu) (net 27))
 (segment (start 130.7846 94.8436) (end 129.7432 93.8022) (width 0.25) (layer F.Cu) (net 27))
 (segment (start 130.7846 108.8136) (end 130.7846 94.8436) (width 0.25) (layer F.Cu) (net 27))
 (segment (start 137.498234 84.310634) (end 138.6332 85.4456) (width 0.25) (layer B.Cu) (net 16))
 (segment (start 124.6378 85.075998) (end 125.403164 84.310634) (width 0.25) (layer B.Cu) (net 16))
 (segment (start 124.6378 109.0344) (end 124.6378 85.075998) (width 0.25) (layer B.Cu) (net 16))
 (segment (start 125.403164 84.310634) (end 137.498234 84.310634) (width 0.25) (layer B.Cu) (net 16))
 (segment (start 126.0856 110.4822) (end 124.6378 109.0344) (width 0.25) (layer B.Cu) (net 16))
 (segment (start 126.0856 111.5822) (end 126.0856 110.4822) (width 0.25) (layer B.Cu) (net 16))
 (segment (start 156.066201 104.731391) (end 149.714791 104.731391) (width 0.25) (layer B.Cu) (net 18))
 (segment (start 145.6436 100.6602) (end 140.0302 100.6602) (width 0.25) (layer B.Cu) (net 18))
 (segment (start 149.714791 104.731391) (end 145.6436 100.6602) (width 0.25) (layer B.Cu) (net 18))
 (segment (start 136.893199 86.245599) (end 136.0932 85.4456) (width 0.25) (layer B.Cu) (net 18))
 (segment (start 140.0302 100.6602) (end 136.271 96.901) (width 0.25) (layer B.Cu) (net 18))
 (segment (start 136.271 96.901) (end 136.271 95.123) (width 0.25) (layer B.Cu) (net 18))
 (segment (start 137.396417 93.997583) (end 137.396417 86.748817) (width 0.25) (layer B.Cu) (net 18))
 (segment (start 136.271 95.123) (end 137.396417 93.997583) (width 0.25) (layer B.Cu) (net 18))
 (segment (start 137.396417 86.748817) (end 136.893199 86.245599) (width 0.25) (layer B.Cu) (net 18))
 (segment (start 159.5882 108.25339) (end 158.90381 107.569) (width 0.25) (layer B.Cu) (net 18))
 (segment (start 159.5882 111.0488) (end 159.5882 108.25339) (width 0.25) (layer B.Cu) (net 18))
 (segment (start 158.90381 107.569) (end 156.066201 104.731391) (width 0.25) (layer B.Cu) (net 18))
 (segment (start 159.131 107.79619) (end 158.90381 107.569) (width 0.25) (layer B.Cu) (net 18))
 (segment (start 131.634599 113.043601) (end 130.7846 113.8936) (width 0.25) (layer B.Cu) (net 3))
 (segment (start 132.2832 112.395) (end 131.634599 113.043601) (width 0.25) (layer B.Cu) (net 3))
 (segment (start 132.2832 96.8756) (end 132.2832 112.395) (width 0.25) (layer B.Cu) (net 3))
 (segment (start 128.4732 93.0656) (end 132.2832 96.8756) (width 0.25) (layer B.Cu) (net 3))
 (segment (start 132.4102 109.728) (end 132.4102 96.14041) (width 0.25) (layer F.Cu) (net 5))
 (segment (start 130.7846 111.3536) (end 132.4102 109.728) (width 0.25) (layer F.Cu) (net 5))
 (segment (start 132.4102 96.14041) (end 131.813199 95.543409) (width 0.25) (layer F.Cu) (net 5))
 (segment (start 131.813199 93.865599) (end 131.0132 93.0656) (width 0.25) (layer F.Cu) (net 5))
 (segment (start 131.813199 95.543409) (end 131.813199 93.865599) (width 0.25) (layer F.Cu) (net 5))
 (segment (start 133.5532 85.217) (end 133.5532 85.4456) (width 0.25) (layer F.Cu) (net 20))
 (segment (start 133.5532 85.2678) (end 133.5532 85.4456) (width 0.25) (layer F.Cu) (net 20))
 (segment (start 136.6774 82.1436) (end 133.5532 85.2678) (width 0.25) (layer F.Cu) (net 20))
 (segment (start 136.6774 81.8896) (end 136.6774 82.1436) (width 0.25) (layer F.Cu) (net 20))
 (segment (start 159.004 85.3948) (end 158.9532 85.4456) (width 0.25) (layer F.Cu) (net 2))
 (segment (start 159.004 81.3054) (end 159.004 85.3948) (width 0.25) (layer F.Cu) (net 2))
 (segment (start 155.2956 84.328) (end 156.4132 85.4456) (width 0.25) (layer F.Cu) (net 4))
 (segment (start 155.2956 81.3054) (end 155.2956 84.328) (width 0.25) (layer F.Cu) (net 4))
 (segment (start 153.02781 84.60021) (end 153.8732 85.4456) (width 0.25) (layer F.Cu) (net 6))
 (segment (start 153.02781 84.2918) (end 153.02781 84.60021) (width 0.25) (layer F.Cu) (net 6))
 (segment (start 151.5364 82.80039) (end 153.02781 84.2918) (width 0.25) (layer F.Cu) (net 6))
 (segment (start 151.5364 81.2927) (end 151.5364 82.80039) (width 0.25) (layer F.Cu) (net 6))
 (segment (start 131.813199 86.245599) (end 131.0132 85.4456) (width 0.25) (layer F.Cu) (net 22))
 (segment (start 132.428199 93.605601) (end 132.428199 86.860599) (width 0.25) (layer F.Cu) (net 22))
 (segment (start 135.4582 110.3376) (end 135.4582 96.635602) (width 0.25) (layer F.Cu) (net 22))
 (segment (start 135.4582 96.635602) (end 132.428199 93.605601) (width 0.25) (layer F.Cu) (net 22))
 (segment (start 132.428199 86.860599) (end 131.813199 86.245599) (width 0.25) (layer F.Cu) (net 22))
 (segment (start 139.954 75.1356) (end 144.454 75.1356) (width 0.25) (layer F.Cu) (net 28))
 (segment (start 134.353199 93.865599) (end 133.5532 93.0656) (width 0.25) (layer F.Cu) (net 7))
 (segment (start 135.908211 95.420611) (end 134.353199 93.865599) (width 0.25) (layer F.Cu) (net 7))
 (segment (start 135.908211 99.586211) (end 135.908211 95.420611) (width 0.25) (layer F.Cu) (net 7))
 (segment (start 142.6464 106.3244) (end 135.908211 99.586211) (width 0.25) (layer F.Cu) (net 7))
 (segment (start 137.5664 97.0026) (end 137.5664 96.1644) (width 0.25) (layer B.Cu) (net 8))
 (segment (start 140.7922 97.917) (end 138.4808 97.917) (width 0.25) (layer B.Cu) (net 8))
 (segment (start 142.494 96.2152) (end 140.7922 97.917) (width 0.25) (layer B.Cu) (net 8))
 (segment (start 138.4808 97.917) (end 137.5664 97.0026) (width 0.25) (layer B.Cu) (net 8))
 (segment (start 142.494 92.4814) (end 142.494 96.2152) (width 0.25) (layer B.Cu) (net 8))
 (segment (start 143.2814 91.694) (end 142.494 92.4814) (width 0.25) (layer B.Cu) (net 8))
 (segment (start 145.0848 91.694) (end 143.2814 91.694) (width 0.25) (layer B.Cu) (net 8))
 (segment (start 151.3332 85.4456) (end 145.0848 91.694) (width 0.25) (layer B.Cu) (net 8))
 (segment (start 136.358222 94.461992) (end 136.0932 94.19697) (width 0.25) (layer F.Cu) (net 9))
 (segment (start 136.358222 97.496222) (end 136.358222 94.461992) (width 0.25) (layer F.Cu) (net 9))
 (segment (start 145.1864 106.3244) (end 136.358222 97.496222) (width 0.25) (layer F.Cu) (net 9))
 (segment (start 136.0932 94.19697) (end 136.0932 93.0656) (width 0.25) (layer F.Cu) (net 9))
 (segment (start 140.868399 107.086399) (end 140.1064 106.3244) (width 0.25) (layer F.Cu) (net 10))
 (segment (start 151.13 107.442) (end 141.224 107.442) (width 0.25) (layer F.Cu) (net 10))
 (segment (start 146.431 100.711) (end 151.638 105.918) (width 0.25) (layer F.Cu) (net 10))
 (segment (start 146.431 94.7928) (end 146.431 100.711) (width 0.25) (layer F.Cu) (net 10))
 (segment (start 151.638 106.934) (end 151.13 107.442) (width 0.25) (layer F.Cu) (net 10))
 (segment (start 147.4724 93.7514) (end 146.431 94.7928) (width 0.25) (layer F.Cu) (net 10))
 (segment (start 151.638 105.918) (end 151.638 106.934) (width 0.25) (layer F.Cu) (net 10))
 (segment (start 147.4724 86.7664) (end 147.4724 93.7514) (width 0.25) (layer F.Cu) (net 10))
 (segment (start 141.224 107.442) (end 140.1064 106.3244) (width 0.25) (layer F.Cu) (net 10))
 (segment (start 148.7932 85.4456) (end 147.4724 86.7664) (width 0.25) (layer F.Cu) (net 10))
 (segment (start 138.811 97.409) (end 147.7264 106.3244) (width 0.25) (layer F.Cu) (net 11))
 (segment (start 138.811 93.472) (end 138.811 97.409) (width 0.25) (layer F.Cu) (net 11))
 (segment (start 138.6332 93.2942) (end 138.811 93.472) (width 0.25) (layer F.Cu) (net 11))
 (segment (start 138.6332 93.0656) (end 138.6332 93.2942) (width 0.25) (layer F.Cu) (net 11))
 (segment (start 151.3332 104.8512) (end 152.8064 106.3244) (width 0.25) (layer F.Cu) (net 19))
 (segment (start 151.3332 93.0656) (end 151.3332 104.8512) (width 0.25) (layer F.Cu) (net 19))
 (segment (start 155.3464 94.5388) (end 155.3464 96.1644) (width 0.25) (layer F.Cu) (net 21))
 (segment (start 153.8732 93.0656) (end 155.3464 94.5388) (width 0.25) (layer F.Cu) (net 21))
 (segment (start 155.613201 93.865599) (end 156.4132 93.0656) (width 0.25) (layer B.Cu) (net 23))
 (segment (start 154.076399 95.402401) (end 155.613201 93.865599) (width 0.25) (layer B.Cu) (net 23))
 (segment (start 148.488399 95.402401) (end 154.076399 95.402401) (width 0.25) (layer B.Cu) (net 23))
 (segment (start 147.7264 96.1644) (end 148.488399 95.402401) (width 0.25) (layer B.Cu) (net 23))
 (segment (start 129.273199 86.245599) (end 128.4732 85.4456) (width 0.25) (layer B.Cu) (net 24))
 (segment (start 132.3086 89.281) (end 129.273199 86.245599) (width 0.25) (layer B.Cu) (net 24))
 (segment (start 132.3086 94.2086) (end 132.3086 89.281) (width 0.25) (layer B.Cu) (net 24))
 (segment (start 139.7 101.6) (end 132.3086 94.2086) (width 0.25) (layer B.Cu) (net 24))
 (segment (start 145.542 101.6) (end 139.7 101.6) (width 0.25) (layer B.Cu) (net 24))
 (segment (start 150.2664 106.3244) (end 145.542 101.6) (width 0.25) (layer B.Cu) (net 24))
 (segment (start 158.9532 94.9198) (end 158.9532 93.0656) (width 0.25) (layer B.Cu) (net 25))
 (segment (start 156.083 97.79) (end 158.9532 94.9198) (width 0.25) (layer B.Cu) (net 25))
 (segment (start 146.812 97.79) (end 156.083 97.79) (width 0.25) (layer B.Cu) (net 25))
 (segment (start 145.1864 96.1644) (end 146.812 97.79) (width 0.25) (layer B.Cu) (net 25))
 (segment (start 154.259399 107.411401) (end 155.3464 106.3244) (width 0.25) (layer B.Cu) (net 26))
 (segment (start 149.744639 107.411401) (end 154.259399 107.411401) (width 0.25) (layer B.Cu) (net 26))
 (segment (start 148.971 106.637762) (end 149.744639 107.411401) (width 0.25) (layer B.Cu) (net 26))
 (segment (start 145.585187 102.616) (end 148.971 106.001813) (width 0.25) (layer B.Cu) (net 26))
 (segment (start 138.898598 102.616) (end 145.585187 102.616) (width 0.25) (layer B.Cu) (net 26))
 (segment (start 129.6924 89.2048) (end 129.6924 93.409802) (width 0.25) (layer B.Cu) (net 26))
 (segment (start 148.971 106.001813) (end 148.971 106.637762) (width 0.25) (layer B.Cu) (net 26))
 (segment (start 129.6924 93.409802) (end 138.898598 102.616) (width 0.25) (layer B.Cu) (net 26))
 (segment (start 125.9332 85.4456) (end 129.6924 89.2048) (width 0.25) (layer B.Cu) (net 26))
 (segment (start 141.9582 110.3376) (end 141.9582 114.8376) (width 0.25) (layer F.Cu) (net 29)))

